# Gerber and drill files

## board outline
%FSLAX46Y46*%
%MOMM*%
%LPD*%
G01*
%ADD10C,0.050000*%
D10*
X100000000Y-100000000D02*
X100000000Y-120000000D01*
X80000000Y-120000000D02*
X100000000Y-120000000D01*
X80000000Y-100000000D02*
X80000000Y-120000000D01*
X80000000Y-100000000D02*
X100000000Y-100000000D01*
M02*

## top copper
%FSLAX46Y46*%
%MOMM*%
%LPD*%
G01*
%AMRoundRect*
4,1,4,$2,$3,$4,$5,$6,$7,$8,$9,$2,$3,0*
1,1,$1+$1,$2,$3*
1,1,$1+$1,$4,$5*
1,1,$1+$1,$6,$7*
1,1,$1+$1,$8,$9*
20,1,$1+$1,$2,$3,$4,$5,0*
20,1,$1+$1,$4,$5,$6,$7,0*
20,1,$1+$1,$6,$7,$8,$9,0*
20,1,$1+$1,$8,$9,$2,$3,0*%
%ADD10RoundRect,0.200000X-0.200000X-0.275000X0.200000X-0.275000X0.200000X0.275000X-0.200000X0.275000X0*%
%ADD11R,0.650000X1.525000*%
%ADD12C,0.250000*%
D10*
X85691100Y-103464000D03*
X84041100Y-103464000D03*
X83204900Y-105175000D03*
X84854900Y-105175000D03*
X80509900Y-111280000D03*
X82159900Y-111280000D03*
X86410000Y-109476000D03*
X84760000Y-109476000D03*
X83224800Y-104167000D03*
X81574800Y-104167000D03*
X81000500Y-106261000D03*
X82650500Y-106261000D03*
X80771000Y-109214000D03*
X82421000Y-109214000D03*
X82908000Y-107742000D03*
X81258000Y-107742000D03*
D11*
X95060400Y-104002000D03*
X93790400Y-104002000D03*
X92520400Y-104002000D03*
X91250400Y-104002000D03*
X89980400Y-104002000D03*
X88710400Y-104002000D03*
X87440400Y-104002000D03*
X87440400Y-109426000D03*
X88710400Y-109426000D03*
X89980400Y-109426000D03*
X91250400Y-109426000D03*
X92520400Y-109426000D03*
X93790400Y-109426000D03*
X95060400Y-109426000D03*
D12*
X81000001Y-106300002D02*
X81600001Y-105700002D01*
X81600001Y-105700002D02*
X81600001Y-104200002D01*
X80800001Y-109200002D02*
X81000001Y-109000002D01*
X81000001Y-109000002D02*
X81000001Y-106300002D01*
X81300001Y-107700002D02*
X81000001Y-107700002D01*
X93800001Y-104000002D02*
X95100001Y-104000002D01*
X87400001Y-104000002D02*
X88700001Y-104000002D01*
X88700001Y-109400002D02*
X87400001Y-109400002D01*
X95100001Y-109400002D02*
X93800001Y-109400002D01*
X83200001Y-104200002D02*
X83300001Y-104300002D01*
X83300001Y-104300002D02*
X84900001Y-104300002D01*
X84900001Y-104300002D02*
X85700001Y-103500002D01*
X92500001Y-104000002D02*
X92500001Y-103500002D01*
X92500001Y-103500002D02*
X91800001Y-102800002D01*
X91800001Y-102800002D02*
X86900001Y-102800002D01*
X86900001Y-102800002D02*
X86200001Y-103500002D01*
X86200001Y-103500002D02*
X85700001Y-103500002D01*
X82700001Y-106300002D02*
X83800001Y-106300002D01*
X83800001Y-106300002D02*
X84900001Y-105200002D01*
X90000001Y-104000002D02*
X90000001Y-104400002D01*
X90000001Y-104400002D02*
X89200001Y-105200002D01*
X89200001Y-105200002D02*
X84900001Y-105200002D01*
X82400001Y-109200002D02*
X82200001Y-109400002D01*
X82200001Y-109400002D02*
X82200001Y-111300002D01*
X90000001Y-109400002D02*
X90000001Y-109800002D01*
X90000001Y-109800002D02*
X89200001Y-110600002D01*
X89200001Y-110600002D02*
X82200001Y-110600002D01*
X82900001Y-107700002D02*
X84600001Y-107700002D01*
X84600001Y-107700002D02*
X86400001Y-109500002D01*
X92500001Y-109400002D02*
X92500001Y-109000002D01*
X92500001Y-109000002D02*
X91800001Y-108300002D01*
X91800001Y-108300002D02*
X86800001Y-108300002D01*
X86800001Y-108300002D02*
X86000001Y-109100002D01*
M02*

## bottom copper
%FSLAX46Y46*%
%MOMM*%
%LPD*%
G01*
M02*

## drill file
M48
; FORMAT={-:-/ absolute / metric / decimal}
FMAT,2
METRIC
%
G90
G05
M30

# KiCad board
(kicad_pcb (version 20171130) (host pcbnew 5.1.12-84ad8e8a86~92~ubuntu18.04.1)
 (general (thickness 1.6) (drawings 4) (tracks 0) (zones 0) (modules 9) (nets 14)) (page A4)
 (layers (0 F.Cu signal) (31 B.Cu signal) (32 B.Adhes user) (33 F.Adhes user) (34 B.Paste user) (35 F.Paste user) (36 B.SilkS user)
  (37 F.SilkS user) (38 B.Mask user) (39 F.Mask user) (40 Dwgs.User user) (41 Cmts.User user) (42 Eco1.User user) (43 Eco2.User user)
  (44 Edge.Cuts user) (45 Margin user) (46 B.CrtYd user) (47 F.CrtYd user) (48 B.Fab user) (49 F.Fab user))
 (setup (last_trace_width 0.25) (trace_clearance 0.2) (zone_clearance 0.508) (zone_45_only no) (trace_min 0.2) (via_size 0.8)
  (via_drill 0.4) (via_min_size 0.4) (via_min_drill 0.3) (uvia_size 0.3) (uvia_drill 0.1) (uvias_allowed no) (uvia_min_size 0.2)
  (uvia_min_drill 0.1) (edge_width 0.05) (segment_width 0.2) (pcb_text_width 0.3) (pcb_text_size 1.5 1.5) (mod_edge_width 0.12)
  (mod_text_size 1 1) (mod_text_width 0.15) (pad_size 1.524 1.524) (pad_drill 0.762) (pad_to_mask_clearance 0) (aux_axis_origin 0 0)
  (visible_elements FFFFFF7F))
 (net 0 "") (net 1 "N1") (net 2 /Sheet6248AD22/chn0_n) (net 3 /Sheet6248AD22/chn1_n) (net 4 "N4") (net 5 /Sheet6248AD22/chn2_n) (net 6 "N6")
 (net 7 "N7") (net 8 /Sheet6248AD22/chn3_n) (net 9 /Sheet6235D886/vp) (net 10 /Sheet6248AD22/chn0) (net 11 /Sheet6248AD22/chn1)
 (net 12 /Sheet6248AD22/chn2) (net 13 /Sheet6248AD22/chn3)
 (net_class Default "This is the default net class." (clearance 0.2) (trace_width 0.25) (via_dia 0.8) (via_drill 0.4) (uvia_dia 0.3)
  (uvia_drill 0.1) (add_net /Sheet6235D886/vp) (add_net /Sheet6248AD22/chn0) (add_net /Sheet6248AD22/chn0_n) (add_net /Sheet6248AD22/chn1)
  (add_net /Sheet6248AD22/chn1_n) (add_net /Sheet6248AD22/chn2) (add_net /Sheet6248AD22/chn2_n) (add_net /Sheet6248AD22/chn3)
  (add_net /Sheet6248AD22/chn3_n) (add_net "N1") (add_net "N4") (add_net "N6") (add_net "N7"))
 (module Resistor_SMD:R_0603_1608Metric (layer F.Cu) (at 84.866100 103.464000)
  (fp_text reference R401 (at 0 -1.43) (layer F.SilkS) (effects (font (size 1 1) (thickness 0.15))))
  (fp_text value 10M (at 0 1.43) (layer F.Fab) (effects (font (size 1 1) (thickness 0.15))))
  (pad 2 smd roundrect (at 0.825 0) (size 0.8 0.95) (layers F.Cu F.Mask F.Paste) (roundrect_rratio 0.25) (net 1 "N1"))
  (pad 1 smd roundrect (at -0.825 0) (size 0.8 0.95) (layers F.Cu F.Mask F.Paste) (roundrect_rratio 0.25) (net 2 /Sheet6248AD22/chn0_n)))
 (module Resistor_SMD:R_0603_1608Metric (layer F.Cu) (at 84.029900 105.175000)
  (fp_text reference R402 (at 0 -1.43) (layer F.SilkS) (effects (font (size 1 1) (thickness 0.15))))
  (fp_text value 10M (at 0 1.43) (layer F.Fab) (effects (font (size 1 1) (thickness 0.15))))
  (pad 1 smd roundrect (at -0.825 0) (size 0.8 0.95) (layers F.Cu F.Mask F.Paste) (roundrect_rratio 0.25) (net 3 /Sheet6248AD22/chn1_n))
  (pad 2 smd roundrect (at 0.825 0) (size 0.8 0.95) (layers F.Cu F.Mask F.Paste) (roundrect_rratio 0.25) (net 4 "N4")))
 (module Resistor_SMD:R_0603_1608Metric (layer F.Cu) (at 81.334900 111.280000)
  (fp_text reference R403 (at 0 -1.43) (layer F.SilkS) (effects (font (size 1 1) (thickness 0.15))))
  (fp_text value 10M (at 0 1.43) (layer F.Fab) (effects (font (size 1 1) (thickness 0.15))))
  (pad 1 smd roundrect (at -0.825 0) (size 0.8 0.95) (layers F.Cu F.Mask F.Paste) (roundrect_rratio 0.25) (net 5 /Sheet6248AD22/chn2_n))
  (pad 2 smd roundrect (at 0.825 0) (size 0.8 0.95) (layers F.Cu F.Mask F.Paste) (roundrect_rratio 0.25) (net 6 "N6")))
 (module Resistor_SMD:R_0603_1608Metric (layer F.Cu) (at 85.585000 109.476000)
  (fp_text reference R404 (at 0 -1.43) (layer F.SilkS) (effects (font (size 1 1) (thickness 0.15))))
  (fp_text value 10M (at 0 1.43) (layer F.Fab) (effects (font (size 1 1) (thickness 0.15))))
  (pad 2 smd roundrect (at 0.825 0) (size 0.8 0.95) (layers F.Cu F.Mask F.Paste) (roundrect_rratio 0.25) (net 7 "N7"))
  (pad 1 smd roundrect (at -0.825 0) (size 0.8 0.95) (layers F.Cu F.Mask F.Paste) (roundrect_rratio 0.25) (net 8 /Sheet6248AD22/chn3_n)))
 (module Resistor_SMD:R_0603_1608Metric (layer F.Cu) (at 82.399800 104.167000)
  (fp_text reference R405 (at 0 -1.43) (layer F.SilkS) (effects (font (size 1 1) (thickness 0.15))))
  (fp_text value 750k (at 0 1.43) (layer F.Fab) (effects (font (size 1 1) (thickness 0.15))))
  (pad 2 smd roundrect (at 0.825 0) (size 0.8 0.95) (layers F.Cu F.Mask F.Paste) (roundrect_rratio 0.25) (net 1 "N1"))
  (pad 1 smd roundrect (at -0.825 0) (size 0.8 0.95) (layers F.Cu F.Mask F.Paste) (roundrect_rratio 0.25) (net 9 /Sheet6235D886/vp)))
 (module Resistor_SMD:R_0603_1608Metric (layer F.Cu) (at 81.825500 106.261000)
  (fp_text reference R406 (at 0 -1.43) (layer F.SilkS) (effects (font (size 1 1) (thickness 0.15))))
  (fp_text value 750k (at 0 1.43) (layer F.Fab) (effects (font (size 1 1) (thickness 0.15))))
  (pad 1 smd roundrect (at -0.825 0) (size 0.8 0.95) (layers F.Cu F.Mask F.Paste) (roundrect_rratio 0.25) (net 9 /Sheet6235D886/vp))
  (pad 2 smd roundrect (at 0.825 0) (size 0.8 0.95) (layers F.Cu F.Mask F.Paste) (roundrect_rratio 0.25) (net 4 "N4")))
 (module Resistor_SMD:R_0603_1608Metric (layer F.Cu) (at 81.596000 109.214000)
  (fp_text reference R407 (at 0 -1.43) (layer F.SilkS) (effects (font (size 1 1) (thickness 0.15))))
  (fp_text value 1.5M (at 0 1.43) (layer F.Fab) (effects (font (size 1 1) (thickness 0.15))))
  (pad 1 smd roundrect (at -0.825 0) (size 0.8 0.95) (layers F.Cu F.Mask F.Paste) (roundrect_rratio 0.25) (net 9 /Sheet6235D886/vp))
  (pad 2 smd roundrect (at 0.825 0) (size 0.8 0.95) (layers F.Cu F.Mask F.Paste) (roundrect_rratio 0.25) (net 6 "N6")))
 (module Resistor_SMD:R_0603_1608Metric (layer F.Cu) (at 82.083000 107.742000)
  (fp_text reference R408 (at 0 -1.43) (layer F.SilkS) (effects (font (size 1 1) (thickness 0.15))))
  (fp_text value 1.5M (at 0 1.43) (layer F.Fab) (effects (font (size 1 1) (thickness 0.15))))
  (pad 2 smd roundrect (at 0.825 0) (size 0.8 0.95) (layers F.Cu F.Mask F.Paste) (roundrect_rratio 0.25) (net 7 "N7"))
  (pad 1 smd roundrect (at -0.825 0) (size 0.8 0.95) (layers F.Cu F.Mask F.Paste) (roundrect_rratio 0.25) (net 9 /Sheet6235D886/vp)))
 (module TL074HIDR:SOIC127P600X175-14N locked (layer F.Cu) (at 91.250400 106.714000 270.000000)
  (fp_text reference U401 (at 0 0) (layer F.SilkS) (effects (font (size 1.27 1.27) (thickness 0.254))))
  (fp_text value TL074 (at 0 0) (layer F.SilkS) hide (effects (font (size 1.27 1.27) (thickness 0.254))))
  (pad 1 smd rect (at -2.712 -3.81) (size 0.65 1.525) (layers F.Cu F.Mask F.Paste) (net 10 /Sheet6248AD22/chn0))
  (pad 2 smd rect (at -2.712 -2.54) (size 0.65 1.525) (layers F.Cu F.Mask F.Paste) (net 10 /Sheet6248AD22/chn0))
  (pad 3 smd rect (at -2.712 -1.27) (size 0.65 1.525) (layers F.Cu F.Mask F.Paste) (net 1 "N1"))
  (pad 4 smd rect (at -2.712 0) (size 0.65 1.525) (layers F.Cu F.Mask F.Paste))
  (pad 5 smd rect (at -2.712 1.27) (size 0.65 1.525) (layers F.Cu F.Mask F.Paste) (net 4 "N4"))
  (pad 6 smd rect (at -2.712 2.54) (size 0.65 1.525) (layers F.Cu F.Mask F.Paste) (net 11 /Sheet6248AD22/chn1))
  (pad 7 smd rect (at -2.712 3.81) (size 0.65 1.525) (layers F.Cu F.Mask F.Paste) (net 11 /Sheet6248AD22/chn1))
  (pad 8 smd rect (at 2.712 3.81) (size 0.65 1.525) (layers F.Cu F.Mask F.Paste) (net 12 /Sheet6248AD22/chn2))
  (pad 9 smd rect (at 2.712 2.54) (size 0.65 1.525) (layers F.Cu F.Mask F.Paste) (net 12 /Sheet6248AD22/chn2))
  (pad 10 smd rect (at 2.712 1.27) (size 0.65 1.525) (layers F.Cu F.Mask F.Paste) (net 6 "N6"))
  (pad 11 smd rect (at 2.712 0) (size 0.65 1.525) (layers F.Cu F.Mask F.Paste))
  (pad 12 smd rect (at 2.712 -1.27) (size 0.65 1.525) (layers F.Cu F.Mask F.Paste) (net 7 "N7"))
  (pad 13 smd rect (at 2.712 -2.54) (size 0.65 1.525) (layers F.Cu F.Mask F.Paste) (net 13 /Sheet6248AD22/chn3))
  (pad 14 smd rect (at 2.712 -3.81) (size 0.65 1.525) (layers F.Cu F.Mask F.Paste) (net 13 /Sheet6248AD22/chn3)))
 (gr_line (start 100 100) (end 100 120) (layer Edge.Cuts) (width 0.05))
 (gr_line (start 80 120) (end 100 120) (layer Edge.Cuts) (width 0.05))
 (gr_line (start 80 100) (end 80 120) (layer Edge.Cuts) (width 0.05))
 (gr_line (start 80 100) (end 100 100) (layer Edge.Cuts) (width 0.05))
 (segment (start 81.000001 106.300002) (end 81.600001 105.700002) (width 0.250000) (layer F.Cu) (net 9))
 (segment (start 81.600001 105.700002) (end 81.600001 104.200002) (width 0.250000) (layer F.Cu) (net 9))
 (segment (start 80.800001 109.200002) (end 81.000001 109.000002) (width 0.250000) (layer F.Cu) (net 9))
 (segment (start 81.000001 109.000002) (end 81.000001 106.300002) (width 0.250000) (layer F.Cu) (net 9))
 (segment (start 81.300001 107.700002) (end 81.000001 107.700002) (width 0.250000) (layer F.Cu) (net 9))
 (segment (start 93.800001 104.000002) (end 95.100001 104.000002) (width 0.250000) (layer F.Cu) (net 10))
 (segment (start 87.400001 104.000002) (end 88.700001 104.000002) (width 0.250000) (layer F.Cu) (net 11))
 (segment (start 88.700001 109.400002) (end 87.400001 109.400002) (width 0.250000) (layer F.Cu) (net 12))
 (segment (start 95.100001 109.400002) (end 93.800001 109.400002) (width 0.250000) (layer F.Cu) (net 13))
 (segment (start 83.200001 104.200002) (end 83.300001 104.300002) (width 0.250000) (layer F.Cu) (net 1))
 (segment (start 83.300001 104.300002) (end 84.900001 104.300002) (width 0.250000) (layer F.Cu) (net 1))
 (segment (start 84.900001 104.300002) (end 85.700001 103.500002) (width 0.250000) (layer F.Cu) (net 1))
 (segment (start 92.500001 104.000002) (end 92.500001 103.500002) (width 0.250000) (layer F.Cu) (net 1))
 (segment (start 92.500001 103.500002) (end 91.800001 102.800002) (width 0.250000) (layer F.Cu) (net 1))
 (segment (start 91.800001 102.800002) (end 86.900001 102.800002) (width 0.250000) (layer F.Cu) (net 1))
 (segment (start 86.900001 102.800002) (end 86.200001 103.500002) (width 0.250000) (layer F.Cu) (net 1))
 (segment (start 86.200001 103.500002) (end 85.700001 103.500002) (width 0.250000) (layer F.Cu) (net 1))
 (segment (start 82.700001 106.300002) (end 83.800001 106.300002) (width 0.250000) (layer F.Cu) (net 4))
 (segment (start 83.800001 106.300002) (end 84.900001 105.200002) (width 0.250000) (layer F.Cu) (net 4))
 (segment (start 90.000001 104.000002) (end 90.000001 104.400002) (width 0.250000) (layer F.Cu) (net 4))
 (segment (start 90.000001 104.400002) (end 89.200001 105.200002) (width 0.250000) (layer F.Cu) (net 4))
 (segment (start 89.200001 105.200002) (end 84.900001 105.200002) (width 0.250000) (layer F.Cu) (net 4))
 (segment (start 82.400001 109.200002) (end 82.200001 109.400002) (width 0.250000) (layer F.Cu) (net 6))
 (segment (start 82.200001 109.400002) (end 82.200001 111.300002) (width 0.250000) (layer F.Cu) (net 6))
 (segment (start 90.000001 109.400002) (end 90.000001 109.800002) (width 0.250000) (layer F.Cu) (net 6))
 (segment (start 90.000001 109.800002) (end 89.200001 110.600002) (width 0.250000) (layer F.Cu) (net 6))
 (segment (start 89.200001 110.600002) (end 82.200001 110.600002) (width 0.250000) (layer F.Cu) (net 6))
 (segment (start 82.900001 107.700002) (end 84.600001 107.700002) (width 0.250000) (layer F.Cu) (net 7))
 (segment (start 84.600001 107.700002) (end 86.400001 109.500002) (width 0.250000) (layer F.Cu) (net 7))
 (segment (start 92.500001 109.400002) (end 92.500001 109.000002) (width 0.250000) (layer F.Cu) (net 7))
 (segment (start 92.500001 109.000002) (end 91.800001 108.300002) (width 0.250000) (layer F.Cu) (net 7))
 (segment (start 91.800001 108.300002) (end 86.800001 108.300002) (width 0.250000) (layer F.Cu) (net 7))
 (segment (start 86.800001 108.300002) (end 86.000001 109.100002) (width 0.250000) (layer F.Cu) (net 7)))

